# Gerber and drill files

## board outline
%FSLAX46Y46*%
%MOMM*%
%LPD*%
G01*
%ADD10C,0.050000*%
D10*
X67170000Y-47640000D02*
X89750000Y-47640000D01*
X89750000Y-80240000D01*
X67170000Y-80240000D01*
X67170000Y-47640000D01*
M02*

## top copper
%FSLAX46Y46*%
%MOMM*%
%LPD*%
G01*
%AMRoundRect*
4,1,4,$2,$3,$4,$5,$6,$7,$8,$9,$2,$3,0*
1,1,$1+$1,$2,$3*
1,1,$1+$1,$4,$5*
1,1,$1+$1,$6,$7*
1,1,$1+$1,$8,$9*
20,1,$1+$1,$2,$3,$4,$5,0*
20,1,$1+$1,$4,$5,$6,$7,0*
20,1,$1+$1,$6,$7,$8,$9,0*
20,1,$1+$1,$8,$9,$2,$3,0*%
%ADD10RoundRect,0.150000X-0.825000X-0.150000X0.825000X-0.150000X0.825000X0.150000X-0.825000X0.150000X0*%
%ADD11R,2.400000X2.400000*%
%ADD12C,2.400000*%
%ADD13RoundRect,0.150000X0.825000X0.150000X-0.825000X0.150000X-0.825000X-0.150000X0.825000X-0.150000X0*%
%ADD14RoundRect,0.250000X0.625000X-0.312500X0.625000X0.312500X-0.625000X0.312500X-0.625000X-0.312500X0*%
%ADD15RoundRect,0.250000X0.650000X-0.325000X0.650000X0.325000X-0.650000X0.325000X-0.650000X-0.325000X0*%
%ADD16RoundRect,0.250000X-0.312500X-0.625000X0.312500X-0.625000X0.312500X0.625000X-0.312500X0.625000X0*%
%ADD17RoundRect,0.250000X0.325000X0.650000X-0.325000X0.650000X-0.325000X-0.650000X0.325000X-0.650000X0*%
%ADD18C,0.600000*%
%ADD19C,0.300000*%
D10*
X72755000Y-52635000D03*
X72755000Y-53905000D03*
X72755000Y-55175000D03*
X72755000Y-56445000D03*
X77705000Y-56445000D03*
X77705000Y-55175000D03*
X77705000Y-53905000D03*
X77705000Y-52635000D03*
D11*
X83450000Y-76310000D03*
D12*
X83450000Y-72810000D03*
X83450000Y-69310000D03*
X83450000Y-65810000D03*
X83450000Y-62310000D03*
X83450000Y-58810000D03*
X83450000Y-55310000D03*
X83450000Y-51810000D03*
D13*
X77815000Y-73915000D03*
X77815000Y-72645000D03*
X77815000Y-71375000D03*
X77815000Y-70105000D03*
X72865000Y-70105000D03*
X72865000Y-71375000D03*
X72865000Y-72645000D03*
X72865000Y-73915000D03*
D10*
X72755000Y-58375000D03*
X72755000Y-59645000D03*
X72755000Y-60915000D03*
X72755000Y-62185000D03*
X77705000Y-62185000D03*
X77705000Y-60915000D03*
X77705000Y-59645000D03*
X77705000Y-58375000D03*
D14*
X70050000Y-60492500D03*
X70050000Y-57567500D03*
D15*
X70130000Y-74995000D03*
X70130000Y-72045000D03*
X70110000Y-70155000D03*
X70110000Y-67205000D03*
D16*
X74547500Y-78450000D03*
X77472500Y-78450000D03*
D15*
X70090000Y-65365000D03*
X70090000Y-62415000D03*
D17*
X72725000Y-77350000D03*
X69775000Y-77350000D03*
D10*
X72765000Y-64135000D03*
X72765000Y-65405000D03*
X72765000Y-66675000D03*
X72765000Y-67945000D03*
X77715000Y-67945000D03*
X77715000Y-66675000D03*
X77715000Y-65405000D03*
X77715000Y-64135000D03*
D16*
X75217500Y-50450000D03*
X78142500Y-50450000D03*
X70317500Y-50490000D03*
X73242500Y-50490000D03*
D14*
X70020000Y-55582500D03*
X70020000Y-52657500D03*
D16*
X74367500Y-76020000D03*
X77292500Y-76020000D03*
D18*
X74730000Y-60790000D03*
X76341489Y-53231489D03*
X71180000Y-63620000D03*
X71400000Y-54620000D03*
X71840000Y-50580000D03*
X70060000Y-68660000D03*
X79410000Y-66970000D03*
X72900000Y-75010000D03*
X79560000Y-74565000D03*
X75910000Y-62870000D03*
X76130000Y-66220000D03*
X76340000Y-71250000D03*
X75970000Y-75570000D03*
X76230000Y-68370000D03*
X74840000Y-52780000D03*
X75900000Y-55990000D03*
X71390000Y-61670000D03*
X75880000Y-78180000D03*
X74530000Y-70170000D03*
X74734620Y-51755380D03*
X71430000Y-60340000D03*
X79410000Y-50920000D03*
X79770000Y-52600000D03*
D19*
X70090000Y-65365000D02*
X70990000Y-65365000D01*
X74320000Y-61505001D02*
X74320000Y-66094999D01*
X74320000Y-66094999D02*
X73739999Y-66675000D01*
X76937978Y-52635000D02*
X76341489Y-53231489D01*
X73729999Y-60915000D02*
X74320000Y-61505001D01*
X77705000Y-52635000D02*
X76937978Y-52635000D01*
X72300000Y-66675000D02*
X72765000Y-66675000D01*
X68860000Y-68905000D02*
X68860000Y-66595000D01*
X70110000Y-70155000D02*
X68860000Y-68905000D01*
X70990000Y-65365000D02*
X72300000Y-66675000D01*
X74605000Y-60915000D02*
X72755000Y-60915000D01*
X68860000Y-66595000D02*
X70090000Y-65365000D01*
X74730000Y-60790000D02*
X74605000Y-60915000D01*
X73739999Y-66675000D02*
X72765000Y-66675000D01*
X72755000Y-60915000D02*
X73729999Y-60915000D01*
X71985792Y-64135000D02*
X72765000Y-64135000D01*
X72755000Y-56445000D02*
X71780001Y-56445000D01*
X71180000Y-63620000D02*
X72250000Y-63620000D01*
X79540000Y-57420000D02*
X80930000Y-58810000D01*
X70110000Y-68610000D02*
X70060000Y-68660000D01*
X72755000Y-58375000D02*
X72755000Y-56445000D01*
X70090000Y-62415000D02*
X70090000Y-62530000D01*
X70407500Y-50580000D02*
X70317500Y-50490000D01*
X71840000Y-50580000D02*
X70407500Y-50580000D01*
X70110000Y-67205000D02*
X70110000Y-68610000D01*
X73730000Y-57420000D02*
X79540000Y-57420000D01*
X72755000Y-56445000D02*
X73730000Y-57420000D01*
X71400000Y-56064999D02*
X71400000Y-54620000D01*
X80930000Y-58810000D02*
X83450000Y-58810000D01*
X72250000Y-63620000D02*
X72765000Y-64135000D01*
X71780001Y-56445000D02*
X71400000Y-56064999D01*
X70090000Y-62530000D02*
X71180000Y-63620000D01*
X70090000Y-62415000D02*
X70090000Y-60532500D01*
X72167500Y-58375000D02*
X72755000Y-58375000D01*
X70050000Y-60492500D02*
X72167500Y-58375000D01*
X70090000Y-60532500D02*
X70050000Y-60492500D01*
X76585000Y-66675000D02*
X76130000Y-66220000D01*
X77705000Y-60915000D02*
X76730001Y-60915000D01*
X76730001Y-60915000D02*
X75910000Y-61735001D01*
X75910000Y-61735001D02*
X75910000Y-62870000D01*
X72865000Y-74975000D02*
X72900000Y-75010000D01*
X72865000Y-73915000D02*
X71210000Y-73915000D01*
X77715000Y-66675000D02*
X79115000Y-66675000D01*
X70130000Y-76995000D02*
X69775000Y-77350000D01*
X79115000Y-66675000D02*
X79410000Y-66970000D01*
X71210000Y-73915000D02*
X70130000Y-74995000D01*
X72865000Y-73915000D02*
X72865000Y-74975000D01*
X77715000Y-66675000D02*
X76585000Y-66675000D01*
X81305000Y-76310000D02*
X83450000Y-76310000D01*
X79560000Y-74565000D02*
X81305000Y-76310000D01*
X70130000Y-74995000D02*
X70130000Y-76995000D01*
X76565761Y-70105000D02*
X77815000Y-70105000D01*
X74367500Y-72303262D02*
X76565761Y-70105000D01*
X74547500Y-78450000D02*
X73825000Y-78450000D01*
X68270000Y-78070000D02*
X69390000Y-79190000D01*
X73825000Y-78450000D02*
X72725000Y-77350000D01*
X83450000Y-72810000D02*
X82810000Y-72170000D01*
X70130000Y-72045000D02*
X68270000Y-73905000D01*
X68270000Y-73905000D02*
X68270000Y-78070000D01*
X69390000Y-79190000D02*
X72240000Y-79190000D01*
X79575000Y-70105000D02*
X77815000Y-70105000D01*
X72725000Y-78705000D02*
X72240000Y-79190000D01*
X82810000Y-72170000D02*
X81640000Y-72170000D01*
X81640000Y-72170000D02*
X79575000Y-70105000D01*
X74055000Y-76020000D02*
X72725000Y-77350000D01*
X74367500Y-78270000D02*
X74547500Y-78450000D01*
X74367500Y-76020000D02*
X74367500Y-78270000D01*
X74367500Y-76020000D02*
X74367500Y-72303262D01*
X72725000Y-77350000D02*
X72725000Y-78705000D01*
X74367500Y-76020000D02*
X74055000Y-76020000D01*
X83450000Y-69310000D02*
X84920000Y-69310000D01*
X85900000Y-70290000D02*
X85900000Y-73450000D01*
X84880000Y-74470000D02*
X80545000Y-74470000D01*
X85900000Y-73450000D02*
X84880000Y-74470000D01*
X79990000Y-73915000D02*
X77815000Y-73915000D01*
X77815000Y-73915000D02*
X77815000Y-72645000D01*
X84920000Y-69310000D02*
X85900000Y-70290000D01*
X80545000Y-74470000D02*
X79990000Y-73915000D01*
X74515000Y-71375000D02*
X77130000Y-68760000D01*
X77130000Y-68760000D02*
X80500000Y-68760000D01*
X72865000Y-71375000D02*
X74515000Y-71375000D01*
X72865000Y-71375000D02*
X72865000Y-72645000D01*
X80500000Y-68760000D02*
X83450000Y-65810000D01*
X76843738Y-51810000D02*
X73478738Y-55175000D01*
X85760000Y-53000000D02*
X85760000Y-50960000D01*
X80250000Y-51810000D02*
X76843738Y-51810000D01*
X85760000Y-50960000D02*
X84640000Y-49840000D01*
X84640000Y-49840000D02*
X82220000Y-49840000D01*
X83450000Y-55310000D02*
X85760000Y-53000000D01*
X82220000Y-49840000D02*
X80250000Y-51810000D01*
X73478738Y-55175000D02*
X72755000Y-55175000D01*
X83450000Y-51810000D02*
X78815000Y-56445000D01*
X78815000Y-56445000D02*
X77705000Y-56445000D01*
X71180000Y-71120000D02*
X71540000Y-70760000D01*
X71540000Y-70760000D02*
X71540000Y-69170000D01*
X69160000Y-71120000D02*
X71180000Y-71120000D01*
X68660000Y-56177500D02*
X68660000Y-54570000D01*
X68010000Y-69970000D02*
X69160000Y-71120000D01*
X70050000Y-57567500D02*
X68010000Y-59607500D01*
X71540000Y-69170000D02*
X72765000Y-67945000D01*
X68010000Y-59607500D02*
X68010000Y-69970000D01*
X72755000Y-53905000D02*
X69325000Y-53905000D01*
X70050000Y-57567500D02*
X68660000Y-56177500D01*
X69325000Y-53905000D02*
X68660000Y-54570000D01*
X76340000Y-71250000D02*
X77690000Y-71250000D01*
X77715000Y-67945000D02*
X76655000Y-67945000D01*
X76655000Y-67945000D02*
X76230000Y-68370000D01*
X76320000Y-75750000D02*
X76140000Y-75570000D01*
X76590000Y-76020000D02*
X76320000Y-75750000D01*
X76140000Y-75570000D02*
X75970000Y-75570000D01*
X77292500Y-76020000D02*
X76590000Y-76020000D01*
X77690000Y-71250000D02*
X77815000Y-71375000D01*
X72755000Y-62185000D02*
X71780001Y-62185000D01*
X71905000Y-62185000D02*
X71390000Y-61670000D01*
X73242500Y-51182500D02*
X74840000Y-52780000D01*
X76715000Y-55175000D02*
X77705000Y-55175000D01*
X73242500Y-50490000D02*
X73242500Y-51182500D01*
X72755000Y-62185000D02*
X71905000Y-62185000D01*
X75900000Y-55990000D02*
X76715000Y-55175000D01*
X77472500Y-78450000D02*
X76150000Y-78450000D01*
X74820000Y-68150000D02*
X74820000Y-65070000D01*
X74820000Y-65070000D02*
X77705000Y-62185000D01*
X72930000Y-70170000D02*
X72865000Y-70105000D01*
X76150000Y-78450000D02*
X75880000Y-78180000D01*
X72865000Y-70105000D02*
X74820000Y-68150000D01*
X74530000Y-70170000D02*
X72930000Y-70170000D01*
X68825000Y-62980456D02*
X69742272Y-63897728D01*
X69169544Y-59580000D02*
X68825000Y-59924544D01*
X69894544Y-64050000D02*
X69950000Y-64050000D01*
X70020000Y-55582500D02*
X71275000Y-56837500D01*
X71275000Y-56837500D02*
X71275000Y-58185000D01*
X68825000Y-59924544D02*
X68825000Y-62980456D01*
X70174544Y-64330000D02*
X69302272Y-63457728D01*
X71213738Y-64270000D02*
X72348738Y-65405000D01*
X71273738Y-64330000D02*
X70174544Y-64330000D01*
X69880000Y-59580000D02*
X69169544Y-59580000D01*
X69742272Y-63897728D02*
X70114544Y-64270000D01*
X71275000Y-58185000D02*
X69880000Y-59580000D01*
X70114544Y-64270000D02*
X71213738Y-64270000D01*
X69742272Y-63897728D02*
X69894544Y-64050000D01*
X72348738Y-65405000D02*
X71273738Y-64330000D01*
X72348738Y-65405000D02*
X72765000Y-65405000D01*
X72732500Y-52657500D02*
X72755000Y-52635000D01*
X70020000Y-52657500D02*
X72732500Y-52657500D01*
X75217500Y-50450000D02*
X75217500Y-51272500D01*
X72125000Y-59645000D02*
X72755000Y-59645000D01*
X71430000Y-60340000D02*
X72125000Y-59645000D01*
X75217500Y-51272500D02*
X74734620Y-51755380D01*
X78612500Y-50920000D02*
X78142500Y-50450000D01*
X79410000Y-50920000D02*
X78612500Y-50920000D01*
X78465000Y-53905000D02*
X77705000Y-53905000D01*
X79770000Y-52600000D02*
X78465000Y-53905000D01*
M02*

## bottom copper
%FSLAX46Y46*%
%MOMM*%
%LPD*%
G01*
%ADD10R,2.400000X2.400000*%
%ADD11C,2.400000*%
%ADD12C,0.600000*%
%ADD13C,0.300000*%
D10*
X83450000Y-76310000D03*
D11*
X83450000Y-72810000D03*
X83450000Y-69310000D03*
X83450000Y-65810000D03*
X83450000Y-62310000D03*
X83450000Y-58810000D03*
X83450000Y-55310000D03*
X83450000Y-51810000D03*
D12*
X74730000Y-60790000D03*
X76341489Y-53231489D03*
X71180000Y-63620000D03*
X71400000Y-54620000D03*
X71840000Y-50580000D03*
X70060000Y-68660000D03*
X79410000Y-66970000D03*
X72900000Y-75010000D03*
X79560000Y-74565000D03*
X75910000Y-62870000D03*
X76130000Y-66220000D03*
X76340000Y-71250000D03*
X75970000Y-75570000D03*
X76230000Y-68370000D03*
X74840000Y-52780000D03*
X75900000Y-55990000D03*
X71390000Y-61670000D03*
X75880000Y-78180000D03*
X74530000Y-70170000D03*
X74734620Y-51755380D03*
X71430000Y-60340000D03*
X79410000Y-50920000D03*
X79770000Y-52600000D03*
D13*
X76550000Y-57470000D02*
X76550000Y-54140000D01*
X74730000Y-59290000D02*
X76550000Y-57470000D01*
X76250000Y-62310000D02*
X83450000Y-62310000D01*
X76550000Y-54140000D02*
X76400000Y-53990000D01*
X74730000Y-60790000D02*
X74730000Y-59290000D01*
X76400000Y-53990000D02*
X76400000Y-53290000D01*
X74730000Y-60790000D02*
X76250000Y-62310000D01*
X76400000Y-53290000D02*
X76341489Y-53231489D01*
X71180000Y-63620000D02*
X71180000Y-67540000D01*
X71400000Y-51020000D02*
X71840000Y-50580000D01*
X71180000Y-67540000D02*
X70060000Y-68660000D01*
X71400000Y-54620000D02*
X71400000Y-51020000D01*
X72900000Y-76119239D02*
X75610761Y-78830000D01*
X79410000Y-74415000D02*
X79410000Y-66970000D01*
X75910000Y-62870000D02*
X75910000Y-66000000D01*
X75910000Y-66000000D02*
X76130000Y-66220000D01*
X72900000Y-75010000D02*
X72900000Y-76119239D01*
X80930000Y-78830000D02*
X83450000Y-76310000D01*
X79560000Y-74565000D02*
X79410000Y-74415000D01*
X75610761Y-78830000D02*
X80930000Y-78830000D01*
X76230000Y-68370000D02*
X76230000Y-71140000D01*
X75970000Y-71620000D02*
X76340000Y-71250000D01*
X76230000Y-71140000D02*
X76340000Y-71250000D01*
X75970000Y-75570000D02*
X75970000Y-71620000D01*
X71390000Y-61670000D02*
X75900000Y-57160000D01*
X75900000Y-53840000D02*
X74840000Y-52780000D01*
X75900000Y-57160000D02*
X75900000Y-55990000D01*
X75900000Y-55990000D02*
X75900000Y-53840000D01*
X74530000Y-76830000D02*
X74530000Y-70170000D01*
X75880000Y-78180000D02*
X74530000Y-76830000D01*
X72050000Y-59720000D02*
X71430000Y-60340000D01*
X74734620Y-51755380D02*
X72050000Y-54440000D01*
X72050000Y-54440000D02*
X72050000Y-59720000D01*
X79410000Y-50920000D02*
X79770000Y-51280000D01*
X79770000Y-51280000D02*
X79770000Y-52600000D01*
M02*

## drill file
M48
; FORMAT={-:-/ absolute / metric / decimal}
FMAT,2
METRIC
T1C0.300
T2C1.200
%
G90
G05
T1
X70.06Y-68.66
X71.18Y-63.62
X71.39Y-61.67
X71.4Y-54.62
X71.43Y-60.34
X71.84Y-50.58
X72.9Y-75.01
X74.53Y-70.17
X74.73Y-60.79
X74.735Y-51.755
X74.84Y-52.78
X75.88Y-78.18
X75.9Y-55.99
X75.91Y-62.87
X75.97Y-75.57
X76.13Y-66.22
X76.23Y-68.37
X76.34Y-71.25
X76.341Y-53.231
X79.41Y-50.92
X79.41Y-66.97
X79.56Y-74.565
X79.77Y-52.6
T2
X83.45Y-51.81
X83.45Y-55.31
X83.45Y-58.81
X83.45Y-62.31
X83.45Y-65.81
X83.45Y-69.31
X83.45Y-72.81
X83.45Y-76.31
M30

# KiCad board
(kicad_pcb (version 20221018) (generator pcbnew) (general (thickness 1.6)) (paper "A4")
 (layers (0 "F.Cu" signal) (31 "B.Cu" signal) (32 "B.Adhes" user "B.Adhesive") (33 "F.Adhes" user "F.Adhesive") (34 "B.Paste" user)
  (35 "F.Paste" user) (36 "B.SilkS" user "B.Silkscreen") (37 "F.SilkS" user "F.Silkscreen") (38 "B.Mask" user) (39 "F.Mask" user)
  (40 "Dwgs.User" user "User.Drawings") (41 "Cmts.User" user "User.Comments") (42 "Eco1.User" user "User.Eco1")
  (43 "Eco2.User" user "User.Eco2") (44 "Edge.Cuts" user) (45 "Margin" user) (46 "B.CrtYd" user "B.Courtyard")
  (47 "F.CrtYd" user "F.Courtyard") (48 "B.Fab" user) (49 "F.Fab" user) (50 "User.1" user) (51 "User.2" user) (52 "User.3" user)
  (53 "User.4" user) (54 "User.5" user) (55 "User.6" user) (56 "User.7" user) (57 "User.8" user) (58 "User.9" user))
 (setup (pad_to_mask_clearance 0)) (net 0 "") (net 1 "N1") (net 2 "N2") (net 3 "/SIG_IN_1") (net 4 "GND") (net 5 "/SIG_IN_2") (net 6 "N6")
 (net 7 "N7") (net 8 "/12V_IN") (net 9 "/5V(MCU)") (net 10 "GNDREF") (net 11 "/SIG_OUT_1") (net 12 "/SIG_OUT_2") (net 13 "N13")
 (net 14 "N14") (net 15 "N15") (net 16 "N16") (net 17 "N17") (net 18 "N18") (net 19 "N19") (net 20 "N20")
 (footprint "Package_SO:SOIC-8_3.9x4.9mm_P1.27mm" (layer "F.Cu") (at 75.23 54.54)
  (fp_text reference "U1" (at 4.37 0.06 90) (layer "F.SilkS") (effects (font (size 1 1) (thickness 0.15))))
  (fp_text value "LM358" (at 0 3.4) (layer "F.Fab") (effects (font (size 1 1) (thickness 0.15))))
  (pad "1" smd roundrect (at -2.475 -1.905) (size 1.95 0.6) (layers "F.Cu" "F.Paste" "F.Mask") (roundrect_rratio 0.25) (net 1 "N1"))
  (pad "2" smd roundrect (at -2.475 -0.635) (size 1.95 0.6) (layers "F.Cu" "F.Paste" "F.Mask") (roundrect_rratio 0.25) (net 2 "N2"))
  (pad "3" smd roundrect (at -2.475 0.635) (size 1.95 0.6) (layers "F.Cu" "F.Paste" "F.Mask") (roundrect_rratio 0.25) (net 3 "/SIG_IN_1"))
  (pad "4" smd roundrect (at -2.475 1.905) (size 1.95 0.6) (layers "F.Cu" "F.Paste" "F.Mask") (roundrect_rratio 0.25) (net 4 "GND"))
  (pad "5" smd roundrect (at 2.475 1.905) (size 1.95 0.6) (layers "F.Cu" "F.Paste" "F.Mask") (roundrect_rratio 0.25) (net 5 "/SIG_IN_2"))
  (pad "6" smd roundrect (at 2.475 0.635) (size 1.95 0.6) (layers "F.Cu" "F.Paste" "F.Mask") (roundrect_rratio 0.25) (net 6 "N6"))
  (pad "7" smd roundrect (at 2.475 -0.635) (size 1.95 0.6) (layers "F.Cu" "F.Paste" "F.Mask") (roundrect_rratio 0.25) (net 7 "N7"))
  (pad "8" smd roundrect (at 2.475 -1.905) (size 1.95 0.6) (layers "F.Cu" "F.Paste" "F.Mask") (roundrect_rratio 0.25) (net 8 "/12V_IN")))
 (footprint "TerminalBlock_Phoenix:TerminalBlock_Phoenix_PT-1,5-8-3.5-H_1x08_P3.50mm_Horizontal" (layer "F.Cu") (at 83.45 76.31 90)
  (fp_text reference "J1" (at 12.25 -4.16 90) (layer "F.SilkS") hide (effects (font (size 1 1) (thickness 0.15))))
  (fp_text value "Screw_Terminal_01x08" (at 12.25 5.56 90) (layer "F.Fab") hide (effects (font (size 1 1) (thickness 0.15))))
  (pad "1" thru_hole rect (at 0 0 90) (size 2.4 2.4) (drill 1.2) (layers "*.Cu" "*.Mask") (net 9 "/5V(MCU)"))
  (pad "2" thru_hole circle (at 3.5 0 90) (size 2.4 2.4) (drill 1.2) (layers "*.Cu" "*.Mask") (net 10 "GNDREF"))
  (pad "3" thru_hole circle (at 7 0 90) (size 2.4 2.4) (drill 1.2) (layers "*.Cu" "*.Mask") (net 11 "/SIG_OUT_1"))
  (pad "4" thru_hole circle (at 10.5 0 90) (size 2.4 2.4) (drill 1.2) (layers "*.Cu" "*.Mask") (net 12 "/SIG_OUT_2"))
  (pad "5" thru_hole circle (at 14 0 90) (size 2.4 2.4) (drill 1.2) (layers "*.Cu" "*.Mask") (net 8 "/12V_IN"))
  (pad "6" thru_hole circle (at 17.5 0 90) (size 2.4 2.4) (drill 1.2) (layers "*.Cu" "*.Mask") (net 4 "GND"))
  (pad "7" thru_hole circle (at 21 0 90) (size 2.4 2.4) (drill 1.2) (layers "*.Cu" "*.Mask") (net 3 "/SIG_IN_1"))
  (pad "8" thru_hole circle (at 24.5 0 90) (size 2.4 2.4) (drill 1.2) (layers "*.Cu" "*.Mask") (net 5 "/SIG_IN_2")))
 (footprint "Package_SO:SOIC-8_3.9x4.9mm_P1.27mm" (layer "F.Cu") (at 75.34 72.01 180)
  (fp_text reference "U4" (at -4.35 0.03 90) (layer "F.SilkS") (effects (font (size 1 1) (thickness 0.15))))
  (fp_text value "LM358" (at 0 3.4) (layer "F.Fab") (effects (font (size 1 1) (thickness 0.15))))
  (pad "1" smd roundrect (at -2.475 -1.905 180) (size 1.95 0.6) (layers "F.Cu" "F.Paste" "F.Mask") (roundrect_rratio 0.25)
   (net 11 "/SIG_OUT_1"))
  (pad "2" smd roundrect (at -2.475 -0.635 180) (size 1.95 0.6) (layers "F.Cu" "F.Paste" "F.Mask") (roundrect_rratio 0.25)
   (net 11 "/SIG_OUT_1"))
  (pad "3" smd roundrect (at -2.475 0.635 180) (size 1.95 0.6) (layers "F.Cu" "F.Paste" "F.Mask") (roundrect_rratio 0.25) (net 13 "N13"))
  (pad "4" smd roundrect (at -2.475 1.905 180) (size 1.95 0.6) (layers "F.Cu" "F.Paste" "F.Mask") (roundrect_rratio 0.25) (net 10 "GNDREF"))
  (pad "5" smd roundrect (at 2.475 1.905 180) (size 1.95 0.6) (layers "F.Cu" "F.Paste" "F.Mask") (roundrect_rratio 0.25) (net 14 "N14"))
  (pad "6" smd roundrect (at 2.475 0.635 180) (size 1.95 0.6) (layers "F.Cu" "F.Paste" "F.Mask") (roundrect_rratio 0.25)
   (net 12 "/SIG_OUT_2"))
  (pad "7" smd roundrect (at 2.475 -0.635 180) (size 1.95 0.6) (layers "F.Cu" "F.Paste" "F.Mask") (roundrect_rratio 0.25)
   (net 12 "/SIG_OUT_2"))
  (pad "8" smd roundrect (at 2.475 -1.905 180) (size 1.95 0.6) (layers "F.Cu" "F.Paste" "F.Mask") (roundrect_rratio 0.25) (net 9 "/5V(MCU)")))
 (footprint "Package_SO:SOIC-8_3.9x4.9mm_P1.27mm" (layer "F.Cu") (at 75.23 60.28)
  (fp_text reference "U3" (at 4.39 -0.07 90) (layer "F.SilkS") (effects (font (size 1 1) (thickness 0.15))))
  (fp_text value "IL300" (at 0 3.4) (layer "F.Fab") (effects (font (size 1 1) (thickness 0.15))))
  (pad "1" smd roundrect (at -2.475 -1.905) (size 1.95 0.6) (layers "F.Cu" "F.Paste" "F.Mask") (roundrect_rratio 0.25) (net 4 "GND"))
  (pad "2" smd roundrect (at -2.475 -0.635) (size 1.95 0.6) (layers "F.Cu" "F.Paste" "F.Mask") (roundrect_rratio 0.25) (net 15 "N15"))
  (pad "3" smd roundrect (at -2.475 0.635) (size 1.95 0.6) (layers "F.Cu" "F.Paste" "F.Mask") (roundrect_rratio 0.25) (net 8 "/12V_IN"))
  (pad "4" smd roundrect (at -2.475 1.905) (size 1.95 0.6) (layers "F.Cu" "F.Paste" "F.Mask") (roundrect_rratio 0.25) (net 6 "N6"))
  (pad "5" smd roundrect (at 2.475 1.905) (size 1.95 0.6) (layers "F.Cu" "F.Paste" "F.Mask") (roundrect_rratio 0.25) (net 14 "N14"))
  (pad "6" smd roundrect (at 2.475 0.635) (size 1.95 0.6) (layers "F.Cu" "F.Paste" "F.Mask") (roundrect_rratio 0.25) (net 9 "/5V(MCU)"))
  (pad "7" smd roundrect (at 2.475 -0.635) (size 1.95 0.6) (layers "F.Cu" "F.Paste" "F.Mask") (roundrect_rratio 0.25) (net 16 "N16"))
  (pad "8" smd roundrect (at 2.475 -1.905) (size 1.95 0.6) (layers "F.Cu" "F.Paste" "F.Mask") (roundrect_rratio 0.25) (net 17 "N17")))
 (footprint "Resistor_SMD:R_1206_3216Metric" (layer "F.Cu") (at 70.05 59.03 90)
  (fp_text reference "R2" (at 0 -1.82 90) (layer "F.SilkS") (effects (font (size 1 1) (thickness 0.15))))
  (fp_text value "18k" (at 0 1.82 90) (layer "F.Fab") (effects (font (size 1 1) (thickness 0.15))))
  (pad "1" smd roundrect (at -1.4625 0 90) (size 1.125 1.75) (layers "F.Cu" "F.Paste" "F.Mask") (roundrect_rratio 0.222222) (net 4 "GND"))
  (pad "2" smd roundrect (at 1.4625 0 90) (size 1.125 1.75) (layers "F.Cu" "F.Paste" "F.Mask") (roundrect_rratio 0.222222) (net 2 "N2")))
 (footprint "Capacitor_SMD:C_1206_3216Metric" (layer "F.Cu") (at 70.13 73.52 90)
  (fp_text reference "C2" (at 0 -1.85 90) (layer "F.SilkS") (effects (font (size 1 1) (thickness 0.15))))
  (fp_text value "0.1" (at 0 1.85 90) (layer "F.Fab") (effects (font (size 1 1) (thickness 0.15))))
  (pad "1" smd roundrect (at -1.475 0 90) (size 1.15 1.8) (layers "F.Cu" "F.Paste" "F.Mask") (roundrect_rratio 0.217391) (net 9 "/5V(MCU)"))
  (pad "2" smd roundrect (at 1.475 0 90) (size 1.15 1.8) (layers "F.Cu" "F.Paste" "F.Mask") (roundrect_rratio 0.217391) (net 10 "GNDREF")))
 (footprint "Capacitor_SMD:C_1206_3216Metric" (layer "F.Cu") (at 70.11 68.68 90)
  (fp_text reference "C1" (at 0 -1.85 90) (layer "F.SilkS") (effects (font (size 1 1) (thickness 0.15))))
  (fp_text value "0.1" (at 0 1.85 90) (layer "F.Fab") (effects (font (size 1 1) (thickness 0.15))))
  (pad "1" smd roundrect (at -1.475 0 90) (size 1.15 1.8) (layers "F.Cu" "F.Paste" "F.Mask") (roundrect_rratio 0.217391) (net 8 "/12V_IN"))
  (pad "2" smd roundrect (at 1.475 0 90) (size 1.15 1.8) (layers "F.Cu" "F.Paste" "F.Mask") (roundrect_rratio 0.217391) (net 4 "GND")))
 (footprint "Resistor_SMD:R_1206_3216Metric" (layer "F.Cu") (at 76.01 78.45)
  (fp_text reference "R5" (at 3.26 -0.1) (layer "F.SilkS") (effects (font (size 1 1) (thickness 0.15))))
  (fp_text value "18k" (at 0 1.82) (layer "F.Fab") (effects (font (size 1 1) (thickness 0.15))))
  (pad "1" smd roundrect (at -1.4625 0) (size 1.125 1.75) (layers "F.Cu" "F.Paste" "F.Mask") (roundrect_rratio 0.222222) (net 10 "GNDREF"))
  (pad "2" smd roundrect (at 1.4625 0) (size 1.125 1.75) (layers "F.Cu" "F.Paste" "F.Mask") (roundrect_rratio 0.222222) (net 14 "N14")))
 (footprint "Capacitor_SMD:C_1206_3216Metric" (layer "F.Cu") (at 70.09 63.89 90)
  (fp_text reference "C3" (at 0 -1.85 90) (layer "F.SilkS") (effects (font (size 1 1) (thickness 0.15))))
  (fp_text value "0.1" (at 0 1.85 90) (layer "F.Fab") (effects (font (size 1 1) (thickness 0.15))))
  (pad "1" smd roundrect (at -1.475 0 90) (size 1.15 1.8) (layers "F.Cu" "F.Paste" "F.Mask") (roundrect_rratio 0.217391) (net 8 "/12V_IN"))
  (pad "2" smd roundrect (at 1.475 0 90) (size 1.15 1.8) (layers "F.Cu" "F.Paste" "F.Mask") (roundrect_rratio 0.217391) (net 4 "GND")))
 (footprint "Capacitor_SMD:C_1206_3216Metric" (layer "F.Cu") (at 71.25 77.35 180)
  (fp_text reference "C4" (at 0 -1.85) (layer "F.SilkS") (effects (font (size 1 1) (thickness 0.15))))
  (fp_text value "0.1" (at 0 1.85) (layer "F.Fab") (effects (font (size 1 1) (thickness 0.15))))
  (pad "1" smd roundrect (at -1.475 0 180) (size 1.15 1.8) (layers "F.Cu" "F.Paste" "F.Mask") (roundrect_rratio 0.217391) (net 10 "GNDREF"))
  (pad "2" smd roundrect (at 1.475 0 180) (size 1.15 1.8) (layers "F.Cu" "F.Paste" "F.Mask") (roundrect_rratio 0.217391) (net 9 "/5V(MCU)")))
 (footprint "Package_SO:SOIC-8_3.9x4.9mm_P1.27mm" (layer "F.Cu") (at 75.24 66.04)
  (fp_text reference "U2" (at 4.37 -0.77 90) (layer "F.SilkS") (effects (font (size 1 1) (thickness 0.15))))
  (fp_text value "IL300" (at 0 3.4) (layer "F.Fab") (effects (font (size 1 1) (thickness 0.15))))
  (pad "1" smd roundrect (at -2.475 -1.905) (size 1.95 0.6) (layers "F.Cu" "F.Paste" "F.Mask") (roundrect_rratio 0.25) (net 4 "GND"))
  (pad "2" smd roundrect (at -2.475 -0.635) (size 1.95 0.6) (layers "F.Cu" "F.Paste" "F.Mask") (roundrect_rratio 0.25) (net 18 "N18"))
  (pad "3" smd roundrect (at -2.475 0.635) (size 1.95 0.6) (layers "F.Cu" "F.Paste" "F.Mask") (roundrect_rratio 0.25) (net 8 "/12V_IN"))
  (pad "4" smd roundrect (at -2.475 1.905) (size 1.95 0.6) (layers "F.Cu" "F.Paste" "F.Mask") (roundrect_rratio 0.25) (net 2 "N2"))
  (pad "5" smd roundrect (at 2.475 1.905) (size 1.95 0.6) (layers "F.Cu" "F.Paste" "F.Mask") (roundrect_rratio 0.25) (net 13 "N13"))
  (pad "6" smd roundrect (at 2.475 0.635) (size 1.95 0.6) (layers "F.Cu" "F.Paste" "F.Mask") (roundrect_rratio 0.25) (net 9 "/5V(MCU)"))
  (pad "7" smd roundrect (at 2.475 -0.635) (size 1.95 0.6) (layers "F.Cu" "F.Paste" "F.Mask") (roundrect_rratio 0.25) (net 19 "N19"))
  (pad "8" smd roundrect (at 2.475 -1.905) (size 1.95 0.6) (layers "F.Cu" "F.Paste" "F.Mask") (roundrect_rratio 0.25) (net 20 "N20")))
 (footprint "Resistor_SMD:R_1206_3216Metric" (layer "F.Cu") (at 76.68 50.45)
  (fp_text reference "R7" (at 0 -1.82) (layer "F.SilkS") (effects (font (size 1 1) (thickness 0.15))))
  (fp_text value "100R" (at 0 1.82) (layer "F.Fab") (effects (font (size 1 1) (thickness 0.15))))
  (pad "1" smd roundrect (at -1.4625 0) (size 1.125 1.75) (layers "F.Cu" "F.Paste" "F.Mask") (roundrect_rratio 0.222222) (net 15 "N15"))
  (pad "2" smd roundrect (at 1.4625 0) (size 1.125 1.75) (layers "F.Cu" "F.Paste" "F.Mask") (roundrect_rratio 0.222222) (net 7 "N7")))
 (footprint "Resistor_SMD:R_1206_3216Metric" (layer "F.Cu") (at 71.78 50.49)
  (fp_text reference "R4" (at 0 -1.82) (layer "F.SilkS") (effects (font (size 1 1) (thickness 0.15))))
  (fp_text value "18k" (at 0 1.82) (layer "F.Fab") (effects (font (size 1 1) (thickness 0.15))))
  (pad "1" smd roundrect (at -1.4625 0) (size 1.125 1.75) (layers "F.Cu" "F.Paste" "F.Mask") (roundrect_rratio 0.222222) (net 4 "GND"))
  (pad "2" smd roundrect (at 1.4625 0) (size 1.125 1.75) (layers "F.Cu" "F.Paste" "F.Mask") (roundrect_rratio 0.222222) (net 6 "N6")))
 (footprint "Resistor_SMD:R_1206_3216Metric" (layer "F.Cu") (at 70.02 54.12 90)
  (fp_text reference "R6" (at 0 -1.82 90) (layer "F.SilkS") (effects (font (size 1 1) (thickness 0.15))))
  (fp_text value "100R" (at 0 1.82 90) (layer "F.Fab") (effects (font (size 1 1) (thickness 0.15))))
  (pad "1" smd roundrect (at -1.4625 0 90) (size 1.125 1.75) (layers "F.Cu" "F.Paste" "F.Mask") (roundrect_rratio 0.222222) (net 18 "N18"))
  (pad "2" smd roundrect (at 1.4625 0 90) (size 1.125 1.75) (layers "F.Cu" "F.Paste" "F.Mask") (roundrect_rratio 0.222222) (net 1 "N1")))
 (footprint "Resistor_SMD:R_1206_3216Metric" (layer "F.Cu") (at 75.83 76.02)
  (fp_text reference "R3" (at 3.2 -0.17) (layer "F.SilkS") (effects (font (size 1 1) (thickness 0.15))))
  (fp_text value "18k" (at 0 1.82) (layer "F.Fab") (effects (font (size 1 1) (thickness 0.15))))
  (pad "1" smd roundrect (at -1.4625 0) (size 1.125 1.75) (layers "F.Cu" "F.Paste" "F.Mask") (roundrect_rratio 0.222222) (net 10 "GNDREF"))
  (pad "2" smd roundrect (at 1.4625 0) (size 1.125 1.75) (layers "F.Cu" "F.Paste" "F.Mask") (roundrect_rratio 0.222222) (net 13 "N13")))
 (gr_rect (start 67.17 47.64) (end 89.75 80.24) (stroke (width 0.05) (type default)) (fill none) (layer "Edge.Cuts"))
 (segment (start 70.09 65.365) (end 70.99 65.365) (width 0.3) (layer "F.Cu") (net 8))
 (segment (start 74.32 61.505001) (end 74.32 66.094999) (width 0.3) (layer "F.Cu") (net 8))
 (segment (start 74.32 66.094999) (end 73.739999 66.675) (width 0.3) (layer "F.Cu") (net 8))
 (segment (start 76.937978 52.635) (end 76.341489 53.231489) (width 0.3) (layer "F.Cu") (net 8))
 (segment (start 73.729999 60.915) (end 74.32 61.505001) (width 0.3) (layer "F.Cu") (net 8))
 (segment (start 77.705 52.635) (end 76.937978 52.635) (width 0.3) (layer "F.Cu") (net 8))
 (segment (start 72.3 66.675) (end 72.765 66.675) (width 0.3) (layer "F.Cu") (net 8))
 (segment (start 68.86 68.905) (end 68.86 66.595) (width 0.3) (layer "F.Cu") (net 8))
 (segment (start 70.11 70.155) (end 68.86 68.905) (width 0.3) (layer "F.Cu") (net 8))
 (segment (start 70.99 65.365) (end 72.3 66.675) (width 0.3) (layer "F.Cu") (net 8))
 (segment (start 74.605 60.915) (end 72.755 60.915) (width 0.3) (layer "F.Cu") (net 8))
 (segment (start 68.86 66.595) (end 70.09 65.365) (width 0.3) (layer "F.Cu") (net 8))
 (segment (start 74.73 60.79) (end 74.605 60.915) (width 0.3) (layer "F.Cu") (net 8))
 (segment (start 73.739999 66.675) (end 72.765 66.675) (width 0.3) (layer "F.Cu") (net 8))
 (segment (start 72.755 60.915) (end 73.729999 60.915) (width 0.3) (layer "F.Cu") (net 8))
 (via (at 74.73 60.79) (size 0.6) (drill 0.3) (layers "F.Cu" "B.Cu") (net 8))
 (via (at 76.341489 53.231489) (size 0.6) (drill 0.3) (layers "F.Cu" "B.Cu") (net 8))
 (segment (start 76.55 57.47) (end 76.55 54.14) (width 0.3) (layer "B.Cu") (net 8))
 (segment (start 74.73 59.29) (end 76.55 57.47) (width 0.3) (layer "B.Cu") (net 8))
 (segment (start 76.25 62.31) (end 83.45 62.31) (width 0.3) (layer "B.Cu") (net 8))
 (segment (start 76.55 54.14) (end 76.4 53.99) (width 0.3) (layer "B.Cu") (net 8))
 (segment (start 74.73 60.79) (end 74.73 59.29) (width 0.3) (layer "B.Cu") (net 8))
 (segment (start 76.4 53.99) (end 76.4 53.29) (width 0.3) (layer "B.Cu") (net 8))
 (segment (start 74.73 60.79) (end 76.25 62.31) (width 0.3) (layer "B.Cu") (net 8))
 (segment (start 76.4 53.29) (end 76.341489 53.231489) (width 0.3) (layer "B.Cu") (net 8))
 (segment (start 71.985792 64.135) (end 72.765 64.135) (width 0.3) (layer "F.Cu") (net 4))
 (segment (start 72.755 56.445) (end 71.780001 56.445) (width 0.3) (layer "F.Cu") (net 4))
 (segment (start 71.18 63.62) (end 72.25 63.62) (width 0.3) (layer "F.Cu") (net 4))
 (segment (start 79.54 57.42) (end 80.93 58.81) (width 0.3) (layer "F.Cu") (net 4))
 (segment (start 70.11 68.61) (end 70.06 68.66) (width 0.3) (layer "F.Cu") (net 4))
 (segment (start 72.755 58.375) (end 72.755 56.445) (width 0.3) (layer "F.Cu") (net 4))
 (segment (start 70.09 62.415) (end 70.09 62.53) (width 0.3) (layer "F.Cu") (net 4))
 (segment (start 70.4075 50.58) (end 70.3175 50.49) (width 0.3) (layer "F.Cu") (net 4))
 (segment (start 71.84 50.58) (end 70.4075 50.58) (width 0.3) (layer "F.Cu") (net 4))
 (segment (start 70.11 67.205) (end 70.11 68.61) (width 0.3) (layer "F.Cu") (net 4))
 (segment (start 73.73 57.42) (end 79.54 57.42) (width 0.3) (layer "F.Cu") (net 4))
 (segment (start 72.755 56.445) (end 73.73 57.42) (width 0.3) (layer "F.Cu") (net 4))
 (segment (start 71.4 56.064999) (end 71.4 54.62) (width 0.3) (layer "F.Cu") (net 4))
 (segment (start 80.93 58.81) (end 83.45 58.81) (width 0.3) (layer "F.Cu") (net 4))
 (segment (start 72.25 63.62) (end 72.765 64.135) (width 0.3) (layer "F.Cu") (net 4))
 (segment (start 71.780001 56.445) (end 71.4 56.064999) (width 0.3) (layer "F.Cu") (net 4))
 (segment (start 70.09 62.53) (end 71.18 63.62) (width 0.3) (layer "F.Cu") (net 4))
 (segment (start 70.09 62.415) (end 70.09 60.5325) (width 0.3) (layer "F.Cu") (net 4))
 (segment (start 72.1675 58.375) (end 72.755 58.375) (width 0.3) (layer "F.Cu") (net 4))
 (segment (start 70.05 60.4925) (end 72.1675 58.375) (width 0.3) (layer "F.Cu") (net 4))
 (segment (start 70.09 60.5325) (end 70.05 60.4925) (width 0.3) (layer "F.Cu") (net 4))
 (via (at 71.18 63.62) (size 0.6) (drill 0.3) (layers "F.Cu" "B.Cu") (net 4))
 (via (at 71.4 54.62) (size 0.6) (drill 0.3) (layers "F.Cu" "B.Cu") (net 4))
 (via (at 71.84 50.58) (size 0.6) (drill 0.3) (layers "F.Cu" "B.Cu") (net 4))
 (via (at 70.06 68.66) (size 0.6) (drill 0.3) (layers "F.Cu" "B.Cu") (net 4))
 (segment (start 71.18 63.62) (end 71.18 67.54) (width 0.3) (layer "B.Cu") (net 4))
 (segment (start 71.4 51.02) (end 71.84 50.58) (width 0.3) (layer "B.Cu") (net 4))
 (segment (start 71.18 67.54) (end 70.06 68.66) (width 0.3) (layer "B.Cu") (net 4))
 (segment (start 71.4 54.62) (end 71.4 51.02) (width 0.3) (layer "B.Cu") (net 4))
 (segment (start 76.585 66.675) (end 76.13 66.22) (width 0.3) (layer "F.Cu") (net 9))
 (segment (start 77.705 60.915) (end 76.730001 60.915) (width 0.3) (layer "F.Cu") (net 9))
 (segment (start 76.730001 60.915) (end 75.91 61.735001) (width 0.3) (layer "F.Cu") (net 9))
 (segment (start 75.91 61.735001) (end 75.91 62.87) (width 0.3) (layer "F.Cu") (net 9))
 (segment (start 72.865 74.975) (end 72.9 75.01) (width 0.3) (layer "F.Cu") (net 9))
 (segment (start 72.865 73.915) (end 71.21 73.915) (width 0.3) (layer "F.Cu") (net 9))
 (segment (start 77.715 66.675) (end 79.115 66.675) (width 0.3) (layer "F.Cu") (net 9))
 (segment (start 70.13 76.995) (end 69.775 77.35) (width 0.3) (layer "F.Cu") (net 9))
 (segment (start 79.115 66.675) (end 79.41 66.97) (width 0.3) (layer "F.Cu") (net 9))
 (segment (start 71.21 73.915) (end 70.13 74.995) (width 0.3) (layer "F.Cu") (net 9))
 (segment (start 72.865 73.915) (end 72.865 74.975) (width 0.3) (layer "F.Cu") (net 9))
 (segment (start 77.715 66.675) (end 76.585 66.675) (width 0.3) (layer "F.Cu") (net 9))
 (segment (start 81.305 76.31) (end 83.45 76.31) (width 0.3) (layer "F.Cu") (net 9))
 (segment (start 79.56 74.565) (end 81.305 76.31) (width 0.3) (layer "F.Cu") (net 9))
 (segment (start 70.13 74.995) (end 70.13 76.995) (width 0.3) (layer "F.Cu") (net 9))
 (via (at 79.41 66.97) (size 0.6) (drill 0.3) (layers "F.Cu" "B.Cu") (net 9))
 (via (at 72.9 75.01) (size 0.6) (drill 0.3) (layers "F.Cu" "B.Cu") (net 9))
 (via (at 79.56 74.565) (size 0.6) (drill 0.3) (layers "F.Cu" "B.Cu") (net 9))
 (via (at 75.91 62.87) (size 0.6) (drill 0.3) (layers "F.Cu" "B.Cu") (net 9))
 (via (at 76.13 66.22) (size 0.6) (drill 0.3) (layers "F.Cu" "B.Cu") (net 9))
 (segment (start 72.9 76.119239) (end 75.610761 78.83) (width 0.3) (layer "B.Cu") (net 9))
 (segment (start 79.41 74.415) (end 79.41 66.97) (width 0.3) (layer "B.Cu") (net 9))
 (segment (start 75.91 62.87) (end 75.91 66) (width 0.3) (layer "B.Cu") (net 9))
 (segment (start 75.91 66) (end 76.13 66.22) (width 0.3) (layer "B.Cu") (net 9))
 (segment (start 72.9 75.01) (end 72.9 76.119239) (width 0.3) (layer "B.Cu") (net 9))
 (segment (start 80.93 78.83) (end 83.45 76.31) (width 0.3) (layer "B.Cu") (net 9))
 (segment (start 79.56 74.565) (end 79.41 74.415) (width 0.3) (layer "B.Cu") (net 9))
 (segment (start 75.610761 78.83) (end 80.93 78.83) (width 0.3) (layer "B.Cu") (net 9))
 (segment (start 76.565761 70.105) (end 77.815 70.105) (width 0.3) (layer "F.Cu") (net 10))
 (segment (start 74.3675 72.303262) (end 76.565761 70.105) (width 0.3) (layer "F.Cu") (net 10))
 (segment (start 74.5475 78.45) (end 73.825 78.45) (width 0.3) (layer "F.Cu") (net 10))
 (segment (start 68.27 78.07) (end 69.39 79.19) (width 0.3) (layer "F.Cu") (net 10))
 (segment (start 73.825 78.45) (end 72.725 77.35) (width 0.3) (layer "F.Cu") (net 10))
 (segment (start 83.45 72.81) (end 82.81 72.17) (width 0.3) (layer "F.Cu") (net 10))
 (segment (start 70.13 72.045) (end 68.27 73.905) (width 0.3) (layer "F.Cu") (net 10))
 (segment (start 68.27 73.905) (end 68.27 78.07) (width 0.3) (layer "F.Cu") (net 10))
 (segment (start 69.39 79.19) (end 72.24 79.19) (width 0.3) (layer "F.Cu") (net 10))
 (segment (start 79.575 70.105) (end 77.815 70.105) (width 0.3) (layer "F.Cu") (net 10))
 (segment (start 72.725 78.705) (end 72.24 79.19) (width 0.3) (layer "F.Cu") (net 10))
 (segment (start 82.81 72.17) (end 81.64 72.17) (width 0.3) (layer "F.Cu") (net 10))
 (segment (start 81.64 72.17) (end 79.575 70.105) (width 0.3) (layer "F.Cu") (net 10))
 (segment (start 74.055 76.02) (end 72.725 77.35) (width 0.3) (layer "F.Cu") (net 10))
 (segment (start 74.3675 78.27) (end 74.5475 78.45) (width 0.3) (layer "F.Cu") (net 10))
 (segment (start 74.3675 76.02) (end 74.3675 78.27) (width 0.3) (layer "F.Cu") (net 10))
 (segment (start 74.3675 76.02) (end 74.3675 72.303262) (width 0.3) (layer "F.Cu") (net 10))
 (segment (start 72.725 77.35) (end 72.725 78.705) (width 0.3) (layer "F.Cu") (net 10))
 (segment (start 74.3675 76.02) (end 74.055 76.02) (width 0.3) (layer "F.Cu") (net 10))
 (segment (start 83.45 69.31) (end 84.92 69.31) (width 0.3) (layer "F.Cu") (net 11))
 (segment (start 85.9 70.29) (end 85.9 73.45) (width 0.3) (layer "F.Cu") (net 11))
 (segment (start 84.88 74.47) (end 80.545 74.47) (width 0.3) (layer "F.Cu") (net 11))
 (segment (start 85.9 73.45) (end 84.88 74.47) (width 0.3) (layer "F.Cu") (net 11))
 (segment (start 79.99 73.915) (end 77.815 73.915) (width 0.3) (layer "F.Cu") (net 11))
 (segment (start 77.815 73.915) (end 77.815 72.645) (width 0.3) (layer "F.Cu") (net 11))
 (segment (start 84.92 69.31) (end 85.9 70.29) (width 0.3) (layer "F.Cu") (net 11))
 (segment (start 80.545 74.47) (end 79.99 73.915) (width 0.3) (layer "F.Cu") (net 11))
 (segment (start 74.515 71.375) (end 77.13 68.76) (width 0.3) (layer "F.Cu") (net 12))
 (segment (start 77.13 68.76) (end 80.5 68.76) (width 0.3) (layer "F.Cu") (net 12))
 (segment (start 72.865 71.375) (end 74.515 71.375) (width 0.3) (layer "F.Cu") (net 12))
 (segment (start 72.865 71.375) (end 72.865 72.645) (width 0.3) (layer "F.Cu") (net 12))
 (segment (start 80.5 68.76) (end 83.45 65.81) (width 0.3) (layer "F.Cu") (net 12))
 (segment (start 76.843738 51.81) (end 73.478738 55.175) (width 0.3) (layer "F.Cu") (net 3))
 (segment (start 85.76 53) (end 85.76 50.96) (width 0.3) (layer "F.Cu") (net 3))
 (segment (start 80.25 51.81) (end 76.843738 51.81) (width 0.3) (layer "F.Cu") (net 3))
 (segment (start 85.76 50.96) (end 84.64 49.84) (width 0.3) (layer "F.Cu") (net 3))
 (segment (start 84.64 49.84) (end 82.22 49.84) (width 0.3) (layer "F.Cu") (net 3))
 (segment (start 83.45 55.31) (end 85.76 53) (width 0.3) (layer "F.Cu") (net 3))
 (segment (start 82.22 49.84) (end 80.25 51.81) (width 0.3) (layer "F.Cu") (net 3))
 (segment (start 73.478738 55.175) (end 72.755 55.175) (width 0.3) (layer "F.Cu") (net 3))
 (segment (start 83.45 51.81) (end 78.815 56.445) (width 0.3) (layer "F.Cu") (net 5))
 (segment (start 78.815 56.445) (end 77.705 56.445) (width 0.3) (layer "F.Cu") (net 5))
 (segment (start 71.18 71.12) (end 71.54 70.76) (width 0.3) (layer "F.Cu") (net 2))
 (segment (start 71.54 70.76) (end 71.54 69.17) (width 0.3) (layer "F.Cu") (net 2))
 (segment (start 69.16 71.12) (end 71.18 71.12) (width 0.3) (layer "F.Cu") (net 2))
 (segment (start 68.66 56.1775) (end 68.66 54.57) (width 0.3) (layer "F.Cu") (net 2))
 (segment (start 68.01 69.97) (end 69.16 71.12) (width 0.3) (layer "F.Cu") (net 2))
 (segment (start 70.05 57.5675) (end 68.01 59.6075) (width 0.3) (layer "F.Cu") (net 2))
 (segment (start 71.54 69.17) (end 72.765 67.945) (width 0.3) (layer "F.Cu") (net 2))
 (segment (start 68.01 59.6075) (end 68.01 69.97) (width 0.3) (layer "F.Cu") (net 2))
 (segment (start 72.755 53.905) (end 69.325 53.905) (width 0.3) (layer "F.Cu") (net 2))
 (segment (start 70.05 57.5675) (end 68.66 56.1775) (width 0.3) (layer "F.Cu") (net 2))
 (segment (start 69.325 53.905) (end 68.66 54.57) (width 0.3) (layer "F.Cu") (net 2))
 (segment (start 76.34 71.25) (end 77.69 71.25) (width 0.3) (layer "F.Cu") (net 13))
 (segment (start 77.715 67.945) (end 76.655 67.945) (width 0.3) (layer "F.Cu") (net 13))
 (segment (start 76.655 67.945) (end 76.23 68.37) (width 0.3) (layer "F.Cu") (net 13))
 (segment (start 76.32 75.75) (end 76.14 75.57) (width 0.3) (layer "F.Cu") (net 13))
 (segment (start 76.59 76.02) (end 76.32 75.75) (width 0.3) (layer "F.Cu") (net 13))
 (segment (start 76.14 75.57) (end 75.97 75.57) (width 0.3) (layer "F.Cu") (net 13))
 (segment (start 77.2925 76.02) (end 76.59 76.02) (width 0.3) (layer "F.Cu") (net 13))
 (segment (start 77.69 71.25) (end 77.815 71.375) (width 0.3) (layer "F.Cu") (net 13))
 (via (at 76.34 71.25) (size 0.6) (drill 0.3) (layers "F.Cu" "B.Cu") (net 13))
 (via (at 75.97 75.57) (size 0.6) (drill 0.3) (layers "F.Cu" "B.Cu") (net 13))
 (via (at 76.23 68.37) (size 0.6) (drill 0.3) (layers "F.Cu" "B.Cu") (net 13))
 (segment (start 76.23 68.37) (end 76.23 71.14) (width 0.3) (layer "B.Cu") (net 13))
 (segment (start 75.97 71.62) (end 76.34 71.25) (width 0.3) (layer "B.Cu") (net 13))
 (segment (start 76.23 71.14) (end 76.34 71.25) (width 0.3) (layer "B.Cu") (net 13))
 (segment (start 75.97 75.57) (end 75.97 71.62) (width 0.3) (layer "B.Cu") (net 13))
 (segment (start 72.755 62.185) (end 71.780001 62.185) (width 0.3) (layer "F.Cu") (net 6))
 (segment (start 71.905 62.185) (end 71.39 61.67) (width 0.3) (layer "F.Cu") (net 6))
 (segment (start 73.2425 51.1825) (end 74.84 52.78) (width 0.3) (layer "F.Cu") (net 6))
 (segment (start 76.715 55.175) (end 77.705 55.175) (width 0.3) (layer "F.Cu") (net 6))
 (segment (start 73.2425 50.49) (end 73.2425 51.1825) (width 0.3) (layer "F.Cu") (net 6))
 (segment (start 72.755 62.185) (end 71.905 62.185) (width 0.3) (layer "F.Cu") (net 6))
 (segment (start 75.9 55.99) (end 76.715 55.175) (width 0.3) (layer "F.Cu") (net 6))
 (via (at 74.84 52.78) (size 0.6) (drill 0.3) (layers "F.Cu" "B.Cu") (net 6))
 (via (at 75.9 55.99) (size 0.6) (drill 0.3) (layers "F.Cu" "B.Cu") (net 6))
 (via (at 71.39 61.67) (size 0.6) (drill 0.3) (layers "F.Cu" "B.Cu") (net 6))
 (segment (start 71.39 61.67) (end 75.9 57.16) (width 0.3) (layer "B.Cu") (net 6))
 (segment (start 75.9 53.84) (end 74.84 52.78) (width 0.3) (layer "B.Cu") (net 6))
 (segment (start 75.9 57.16) (end 75.9 55.99) (width 0.3) (layer "B.Cu") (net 6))
 (segment (start 75.9 55.99) (end 75.9 53.84) (width 0.3) (layer "B.Cu") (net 6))
 (segment (start 77.4725 78.45) (end 76.15 78.45) (width 0.3) (layer "F.Cu") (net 14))
 (segment (start 74.82 68.15) (end 74.82 65.07) (width 0.3) (layer "F.Cu") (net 14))
 (segment (start 74.82 65.07) (end 77.705 62.185) (width 0.3) (layer "F.Cu") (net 14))
 (segment (start 72.93 70.17) (end 72.865 70.105) (width 0.3) (layer "F.Cu") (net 14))
 (segment (start 76.15 78.45) (end 75.88 78.18) (width 0.3) (layer "F.Cu") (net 14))
 (segment (start 72.865 70.105) (end 74.82 68.15) (width 0.3) (layer "F.Cu") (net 14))
 (segment (start 74.53 70.17) (end 72.93 70.17) (width 0.3) (layer "F.Cu") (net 14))
 (via (at 75.88 78.18) (size 0.6) (drill 0.3) (layers "F.Cu" "B.Cu") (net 14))
 (via (at 74.53 70.17) (size 0.6) (drill 0.3) (layers "F.Cu" "B.Cu") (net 14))
 (segment (start 74.53 76.83) (end 74.53 70.17) (width 0.3) (layer "B.Cu") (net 14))
 (segment (start 75.88 78.18) (end 74.53 76.83) (width 0.3) (layer "B.Cu") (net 14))
 (segment (start 68.825 62.980456) (end 69.742272 63.897728) (width 0.3) (layer "F.Cu") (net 18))
 (segment (start 69.169544 59.58) (end 68.825 59.924544) (width 0.3) (layer "F.Cu") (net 18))
 (segment (start 69.894544 64.05) (end 69.95 64.05) (width 0.3) (layer "F.Cu") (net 18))
 (segment (start 70.02 55.5825) (end 71.275 56.8375) (width 0.3) (layer "F.Cu") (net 18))
 (segment (start 71.275 56.8375) (end 71.275 58.185) (width 0.3) (layer "F.Cu") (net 18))
 (segment (start 68.825 59.924544) (end 68.825 62.980456) (width 0.3) (layer "F.Cu") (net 18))
 (segment (start 70.174544 64.33) (end 69.302272 63.457728) (width 0.3) (layer "F.Cu") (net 18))
 (segment (start 71.213738 64.27) (end 72.348738 65.405) (width 0.3) (layer "F.Cu") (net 18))
 (segment (start 71.273738 64.33) (end 70.174544 64.33) (width 0.3) (layer "F.Cu") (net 18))
 (segment (start 69.88 59.58) (end 69.169544 59.58) (width 0.3) (layer "F.Cu") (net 18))
 (segment (start 69.742272 63.897728) (end 70.114544 64.27) (width 0.3) (layer "F.Cu") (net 18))
 (segment (start 71.275 58.185) (end 69.88 59.58) (width 0.3) (layer "F.Cu") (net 18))
 (segment (start 70.114544 64.27) (end 71.213738 64.27) (width 0.3) (layer "F.Cu") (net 18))
 (segment (start 69.742272 63.897728) (end 69.894544 64.05) (width 0.3) (layer "F.Cu") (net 18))
 (segment (start 72.348738 65.405) (end 71.273738 64.33) (width 0.3) (layer "F.Cu") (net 18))
 (segment (start 72.348738 65.405) (end 72.765 65.405) (width 0.3) (layer "F.Cu") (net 18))
 (segment (start 72.7325 52.6575) (end 72.755 52.635) (width 0.3) (layer "F.Cu") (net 1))
 (segment (start 70.02 52.6575) (end 72.7325 52.6575) (width 0.3) (layer "F.Cu") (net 1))
 (segment (start 75.2175 50.45) (end 75.2175 51.2725) (width 0.3) (layer "F.Cu") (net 15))
 (segment (start 72.125 59.645) (end 72.755 59.645) (width 0.3) (layer "F.Cu") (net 15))
 (segment (start 71.43 60.34) (end 72.125 59.645) (width 0.3) (layer "F.Cu") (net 15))
 (segment (start 75.2175 51.2725) (end 74.73462 51.75538) (width 0.3) (layer "F.Cu") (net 15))
 (via (at 74.73462 51.75538) (size 0.6) (drill 0.3) (layers "F.Cu" "B.Cu") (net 15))
 (via (at 71.43 60.34) (size 0.6) (drill 0.3) (layers "F.Cu" "B.Cu") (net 15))
 (segment (start 72.05 59.72) (end 71.43 60.34) (width 0.3) (layer "B.Cu") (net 15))
 (segment (start 74.73462 51.75538) (end 72.05 54.44) (width 0.3) (layer "B.Cu") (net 15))
 (segment (start 72.05 54.44) (end 72.05 59.72) (width 0.3) (layer "B.Cu") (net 15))
 (segment (start 78.6125 50.92) (end 78.1425 50.45) (width 0.3) (layer "F.Cu") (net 7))
 (segment (start 79.41 50.92) (end 78.6125 50.92) (width 0.3) (layer "F.Cu") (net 7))
 (segment (start 78.465 53.905) (end 77.705 53.905) (width 0.3) (layer "F.Cu") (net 7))
 (segment (start 79.77 52.6) (end 78.465 53.905) (width 0.3) (layer "F.Cu") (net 7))
 (via (at 79.41 50.92) (size 0.6) (drill 0.3) (layers "F.Cu" "B.Cu") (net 7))
 (via (at 79.77 52.6) (size 0.6) (drill 0.3) (layers "F.Cu" "B.Cu") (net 7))
 (segment (start 79.41 50.92) (end 79.77 51.28) (width 0.3) (layer "B.Cu") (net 7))
 (segment (start 79.77 51.28) (end 79.77 52.6) (width 0.3) (layer "B.Cu") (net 7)))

